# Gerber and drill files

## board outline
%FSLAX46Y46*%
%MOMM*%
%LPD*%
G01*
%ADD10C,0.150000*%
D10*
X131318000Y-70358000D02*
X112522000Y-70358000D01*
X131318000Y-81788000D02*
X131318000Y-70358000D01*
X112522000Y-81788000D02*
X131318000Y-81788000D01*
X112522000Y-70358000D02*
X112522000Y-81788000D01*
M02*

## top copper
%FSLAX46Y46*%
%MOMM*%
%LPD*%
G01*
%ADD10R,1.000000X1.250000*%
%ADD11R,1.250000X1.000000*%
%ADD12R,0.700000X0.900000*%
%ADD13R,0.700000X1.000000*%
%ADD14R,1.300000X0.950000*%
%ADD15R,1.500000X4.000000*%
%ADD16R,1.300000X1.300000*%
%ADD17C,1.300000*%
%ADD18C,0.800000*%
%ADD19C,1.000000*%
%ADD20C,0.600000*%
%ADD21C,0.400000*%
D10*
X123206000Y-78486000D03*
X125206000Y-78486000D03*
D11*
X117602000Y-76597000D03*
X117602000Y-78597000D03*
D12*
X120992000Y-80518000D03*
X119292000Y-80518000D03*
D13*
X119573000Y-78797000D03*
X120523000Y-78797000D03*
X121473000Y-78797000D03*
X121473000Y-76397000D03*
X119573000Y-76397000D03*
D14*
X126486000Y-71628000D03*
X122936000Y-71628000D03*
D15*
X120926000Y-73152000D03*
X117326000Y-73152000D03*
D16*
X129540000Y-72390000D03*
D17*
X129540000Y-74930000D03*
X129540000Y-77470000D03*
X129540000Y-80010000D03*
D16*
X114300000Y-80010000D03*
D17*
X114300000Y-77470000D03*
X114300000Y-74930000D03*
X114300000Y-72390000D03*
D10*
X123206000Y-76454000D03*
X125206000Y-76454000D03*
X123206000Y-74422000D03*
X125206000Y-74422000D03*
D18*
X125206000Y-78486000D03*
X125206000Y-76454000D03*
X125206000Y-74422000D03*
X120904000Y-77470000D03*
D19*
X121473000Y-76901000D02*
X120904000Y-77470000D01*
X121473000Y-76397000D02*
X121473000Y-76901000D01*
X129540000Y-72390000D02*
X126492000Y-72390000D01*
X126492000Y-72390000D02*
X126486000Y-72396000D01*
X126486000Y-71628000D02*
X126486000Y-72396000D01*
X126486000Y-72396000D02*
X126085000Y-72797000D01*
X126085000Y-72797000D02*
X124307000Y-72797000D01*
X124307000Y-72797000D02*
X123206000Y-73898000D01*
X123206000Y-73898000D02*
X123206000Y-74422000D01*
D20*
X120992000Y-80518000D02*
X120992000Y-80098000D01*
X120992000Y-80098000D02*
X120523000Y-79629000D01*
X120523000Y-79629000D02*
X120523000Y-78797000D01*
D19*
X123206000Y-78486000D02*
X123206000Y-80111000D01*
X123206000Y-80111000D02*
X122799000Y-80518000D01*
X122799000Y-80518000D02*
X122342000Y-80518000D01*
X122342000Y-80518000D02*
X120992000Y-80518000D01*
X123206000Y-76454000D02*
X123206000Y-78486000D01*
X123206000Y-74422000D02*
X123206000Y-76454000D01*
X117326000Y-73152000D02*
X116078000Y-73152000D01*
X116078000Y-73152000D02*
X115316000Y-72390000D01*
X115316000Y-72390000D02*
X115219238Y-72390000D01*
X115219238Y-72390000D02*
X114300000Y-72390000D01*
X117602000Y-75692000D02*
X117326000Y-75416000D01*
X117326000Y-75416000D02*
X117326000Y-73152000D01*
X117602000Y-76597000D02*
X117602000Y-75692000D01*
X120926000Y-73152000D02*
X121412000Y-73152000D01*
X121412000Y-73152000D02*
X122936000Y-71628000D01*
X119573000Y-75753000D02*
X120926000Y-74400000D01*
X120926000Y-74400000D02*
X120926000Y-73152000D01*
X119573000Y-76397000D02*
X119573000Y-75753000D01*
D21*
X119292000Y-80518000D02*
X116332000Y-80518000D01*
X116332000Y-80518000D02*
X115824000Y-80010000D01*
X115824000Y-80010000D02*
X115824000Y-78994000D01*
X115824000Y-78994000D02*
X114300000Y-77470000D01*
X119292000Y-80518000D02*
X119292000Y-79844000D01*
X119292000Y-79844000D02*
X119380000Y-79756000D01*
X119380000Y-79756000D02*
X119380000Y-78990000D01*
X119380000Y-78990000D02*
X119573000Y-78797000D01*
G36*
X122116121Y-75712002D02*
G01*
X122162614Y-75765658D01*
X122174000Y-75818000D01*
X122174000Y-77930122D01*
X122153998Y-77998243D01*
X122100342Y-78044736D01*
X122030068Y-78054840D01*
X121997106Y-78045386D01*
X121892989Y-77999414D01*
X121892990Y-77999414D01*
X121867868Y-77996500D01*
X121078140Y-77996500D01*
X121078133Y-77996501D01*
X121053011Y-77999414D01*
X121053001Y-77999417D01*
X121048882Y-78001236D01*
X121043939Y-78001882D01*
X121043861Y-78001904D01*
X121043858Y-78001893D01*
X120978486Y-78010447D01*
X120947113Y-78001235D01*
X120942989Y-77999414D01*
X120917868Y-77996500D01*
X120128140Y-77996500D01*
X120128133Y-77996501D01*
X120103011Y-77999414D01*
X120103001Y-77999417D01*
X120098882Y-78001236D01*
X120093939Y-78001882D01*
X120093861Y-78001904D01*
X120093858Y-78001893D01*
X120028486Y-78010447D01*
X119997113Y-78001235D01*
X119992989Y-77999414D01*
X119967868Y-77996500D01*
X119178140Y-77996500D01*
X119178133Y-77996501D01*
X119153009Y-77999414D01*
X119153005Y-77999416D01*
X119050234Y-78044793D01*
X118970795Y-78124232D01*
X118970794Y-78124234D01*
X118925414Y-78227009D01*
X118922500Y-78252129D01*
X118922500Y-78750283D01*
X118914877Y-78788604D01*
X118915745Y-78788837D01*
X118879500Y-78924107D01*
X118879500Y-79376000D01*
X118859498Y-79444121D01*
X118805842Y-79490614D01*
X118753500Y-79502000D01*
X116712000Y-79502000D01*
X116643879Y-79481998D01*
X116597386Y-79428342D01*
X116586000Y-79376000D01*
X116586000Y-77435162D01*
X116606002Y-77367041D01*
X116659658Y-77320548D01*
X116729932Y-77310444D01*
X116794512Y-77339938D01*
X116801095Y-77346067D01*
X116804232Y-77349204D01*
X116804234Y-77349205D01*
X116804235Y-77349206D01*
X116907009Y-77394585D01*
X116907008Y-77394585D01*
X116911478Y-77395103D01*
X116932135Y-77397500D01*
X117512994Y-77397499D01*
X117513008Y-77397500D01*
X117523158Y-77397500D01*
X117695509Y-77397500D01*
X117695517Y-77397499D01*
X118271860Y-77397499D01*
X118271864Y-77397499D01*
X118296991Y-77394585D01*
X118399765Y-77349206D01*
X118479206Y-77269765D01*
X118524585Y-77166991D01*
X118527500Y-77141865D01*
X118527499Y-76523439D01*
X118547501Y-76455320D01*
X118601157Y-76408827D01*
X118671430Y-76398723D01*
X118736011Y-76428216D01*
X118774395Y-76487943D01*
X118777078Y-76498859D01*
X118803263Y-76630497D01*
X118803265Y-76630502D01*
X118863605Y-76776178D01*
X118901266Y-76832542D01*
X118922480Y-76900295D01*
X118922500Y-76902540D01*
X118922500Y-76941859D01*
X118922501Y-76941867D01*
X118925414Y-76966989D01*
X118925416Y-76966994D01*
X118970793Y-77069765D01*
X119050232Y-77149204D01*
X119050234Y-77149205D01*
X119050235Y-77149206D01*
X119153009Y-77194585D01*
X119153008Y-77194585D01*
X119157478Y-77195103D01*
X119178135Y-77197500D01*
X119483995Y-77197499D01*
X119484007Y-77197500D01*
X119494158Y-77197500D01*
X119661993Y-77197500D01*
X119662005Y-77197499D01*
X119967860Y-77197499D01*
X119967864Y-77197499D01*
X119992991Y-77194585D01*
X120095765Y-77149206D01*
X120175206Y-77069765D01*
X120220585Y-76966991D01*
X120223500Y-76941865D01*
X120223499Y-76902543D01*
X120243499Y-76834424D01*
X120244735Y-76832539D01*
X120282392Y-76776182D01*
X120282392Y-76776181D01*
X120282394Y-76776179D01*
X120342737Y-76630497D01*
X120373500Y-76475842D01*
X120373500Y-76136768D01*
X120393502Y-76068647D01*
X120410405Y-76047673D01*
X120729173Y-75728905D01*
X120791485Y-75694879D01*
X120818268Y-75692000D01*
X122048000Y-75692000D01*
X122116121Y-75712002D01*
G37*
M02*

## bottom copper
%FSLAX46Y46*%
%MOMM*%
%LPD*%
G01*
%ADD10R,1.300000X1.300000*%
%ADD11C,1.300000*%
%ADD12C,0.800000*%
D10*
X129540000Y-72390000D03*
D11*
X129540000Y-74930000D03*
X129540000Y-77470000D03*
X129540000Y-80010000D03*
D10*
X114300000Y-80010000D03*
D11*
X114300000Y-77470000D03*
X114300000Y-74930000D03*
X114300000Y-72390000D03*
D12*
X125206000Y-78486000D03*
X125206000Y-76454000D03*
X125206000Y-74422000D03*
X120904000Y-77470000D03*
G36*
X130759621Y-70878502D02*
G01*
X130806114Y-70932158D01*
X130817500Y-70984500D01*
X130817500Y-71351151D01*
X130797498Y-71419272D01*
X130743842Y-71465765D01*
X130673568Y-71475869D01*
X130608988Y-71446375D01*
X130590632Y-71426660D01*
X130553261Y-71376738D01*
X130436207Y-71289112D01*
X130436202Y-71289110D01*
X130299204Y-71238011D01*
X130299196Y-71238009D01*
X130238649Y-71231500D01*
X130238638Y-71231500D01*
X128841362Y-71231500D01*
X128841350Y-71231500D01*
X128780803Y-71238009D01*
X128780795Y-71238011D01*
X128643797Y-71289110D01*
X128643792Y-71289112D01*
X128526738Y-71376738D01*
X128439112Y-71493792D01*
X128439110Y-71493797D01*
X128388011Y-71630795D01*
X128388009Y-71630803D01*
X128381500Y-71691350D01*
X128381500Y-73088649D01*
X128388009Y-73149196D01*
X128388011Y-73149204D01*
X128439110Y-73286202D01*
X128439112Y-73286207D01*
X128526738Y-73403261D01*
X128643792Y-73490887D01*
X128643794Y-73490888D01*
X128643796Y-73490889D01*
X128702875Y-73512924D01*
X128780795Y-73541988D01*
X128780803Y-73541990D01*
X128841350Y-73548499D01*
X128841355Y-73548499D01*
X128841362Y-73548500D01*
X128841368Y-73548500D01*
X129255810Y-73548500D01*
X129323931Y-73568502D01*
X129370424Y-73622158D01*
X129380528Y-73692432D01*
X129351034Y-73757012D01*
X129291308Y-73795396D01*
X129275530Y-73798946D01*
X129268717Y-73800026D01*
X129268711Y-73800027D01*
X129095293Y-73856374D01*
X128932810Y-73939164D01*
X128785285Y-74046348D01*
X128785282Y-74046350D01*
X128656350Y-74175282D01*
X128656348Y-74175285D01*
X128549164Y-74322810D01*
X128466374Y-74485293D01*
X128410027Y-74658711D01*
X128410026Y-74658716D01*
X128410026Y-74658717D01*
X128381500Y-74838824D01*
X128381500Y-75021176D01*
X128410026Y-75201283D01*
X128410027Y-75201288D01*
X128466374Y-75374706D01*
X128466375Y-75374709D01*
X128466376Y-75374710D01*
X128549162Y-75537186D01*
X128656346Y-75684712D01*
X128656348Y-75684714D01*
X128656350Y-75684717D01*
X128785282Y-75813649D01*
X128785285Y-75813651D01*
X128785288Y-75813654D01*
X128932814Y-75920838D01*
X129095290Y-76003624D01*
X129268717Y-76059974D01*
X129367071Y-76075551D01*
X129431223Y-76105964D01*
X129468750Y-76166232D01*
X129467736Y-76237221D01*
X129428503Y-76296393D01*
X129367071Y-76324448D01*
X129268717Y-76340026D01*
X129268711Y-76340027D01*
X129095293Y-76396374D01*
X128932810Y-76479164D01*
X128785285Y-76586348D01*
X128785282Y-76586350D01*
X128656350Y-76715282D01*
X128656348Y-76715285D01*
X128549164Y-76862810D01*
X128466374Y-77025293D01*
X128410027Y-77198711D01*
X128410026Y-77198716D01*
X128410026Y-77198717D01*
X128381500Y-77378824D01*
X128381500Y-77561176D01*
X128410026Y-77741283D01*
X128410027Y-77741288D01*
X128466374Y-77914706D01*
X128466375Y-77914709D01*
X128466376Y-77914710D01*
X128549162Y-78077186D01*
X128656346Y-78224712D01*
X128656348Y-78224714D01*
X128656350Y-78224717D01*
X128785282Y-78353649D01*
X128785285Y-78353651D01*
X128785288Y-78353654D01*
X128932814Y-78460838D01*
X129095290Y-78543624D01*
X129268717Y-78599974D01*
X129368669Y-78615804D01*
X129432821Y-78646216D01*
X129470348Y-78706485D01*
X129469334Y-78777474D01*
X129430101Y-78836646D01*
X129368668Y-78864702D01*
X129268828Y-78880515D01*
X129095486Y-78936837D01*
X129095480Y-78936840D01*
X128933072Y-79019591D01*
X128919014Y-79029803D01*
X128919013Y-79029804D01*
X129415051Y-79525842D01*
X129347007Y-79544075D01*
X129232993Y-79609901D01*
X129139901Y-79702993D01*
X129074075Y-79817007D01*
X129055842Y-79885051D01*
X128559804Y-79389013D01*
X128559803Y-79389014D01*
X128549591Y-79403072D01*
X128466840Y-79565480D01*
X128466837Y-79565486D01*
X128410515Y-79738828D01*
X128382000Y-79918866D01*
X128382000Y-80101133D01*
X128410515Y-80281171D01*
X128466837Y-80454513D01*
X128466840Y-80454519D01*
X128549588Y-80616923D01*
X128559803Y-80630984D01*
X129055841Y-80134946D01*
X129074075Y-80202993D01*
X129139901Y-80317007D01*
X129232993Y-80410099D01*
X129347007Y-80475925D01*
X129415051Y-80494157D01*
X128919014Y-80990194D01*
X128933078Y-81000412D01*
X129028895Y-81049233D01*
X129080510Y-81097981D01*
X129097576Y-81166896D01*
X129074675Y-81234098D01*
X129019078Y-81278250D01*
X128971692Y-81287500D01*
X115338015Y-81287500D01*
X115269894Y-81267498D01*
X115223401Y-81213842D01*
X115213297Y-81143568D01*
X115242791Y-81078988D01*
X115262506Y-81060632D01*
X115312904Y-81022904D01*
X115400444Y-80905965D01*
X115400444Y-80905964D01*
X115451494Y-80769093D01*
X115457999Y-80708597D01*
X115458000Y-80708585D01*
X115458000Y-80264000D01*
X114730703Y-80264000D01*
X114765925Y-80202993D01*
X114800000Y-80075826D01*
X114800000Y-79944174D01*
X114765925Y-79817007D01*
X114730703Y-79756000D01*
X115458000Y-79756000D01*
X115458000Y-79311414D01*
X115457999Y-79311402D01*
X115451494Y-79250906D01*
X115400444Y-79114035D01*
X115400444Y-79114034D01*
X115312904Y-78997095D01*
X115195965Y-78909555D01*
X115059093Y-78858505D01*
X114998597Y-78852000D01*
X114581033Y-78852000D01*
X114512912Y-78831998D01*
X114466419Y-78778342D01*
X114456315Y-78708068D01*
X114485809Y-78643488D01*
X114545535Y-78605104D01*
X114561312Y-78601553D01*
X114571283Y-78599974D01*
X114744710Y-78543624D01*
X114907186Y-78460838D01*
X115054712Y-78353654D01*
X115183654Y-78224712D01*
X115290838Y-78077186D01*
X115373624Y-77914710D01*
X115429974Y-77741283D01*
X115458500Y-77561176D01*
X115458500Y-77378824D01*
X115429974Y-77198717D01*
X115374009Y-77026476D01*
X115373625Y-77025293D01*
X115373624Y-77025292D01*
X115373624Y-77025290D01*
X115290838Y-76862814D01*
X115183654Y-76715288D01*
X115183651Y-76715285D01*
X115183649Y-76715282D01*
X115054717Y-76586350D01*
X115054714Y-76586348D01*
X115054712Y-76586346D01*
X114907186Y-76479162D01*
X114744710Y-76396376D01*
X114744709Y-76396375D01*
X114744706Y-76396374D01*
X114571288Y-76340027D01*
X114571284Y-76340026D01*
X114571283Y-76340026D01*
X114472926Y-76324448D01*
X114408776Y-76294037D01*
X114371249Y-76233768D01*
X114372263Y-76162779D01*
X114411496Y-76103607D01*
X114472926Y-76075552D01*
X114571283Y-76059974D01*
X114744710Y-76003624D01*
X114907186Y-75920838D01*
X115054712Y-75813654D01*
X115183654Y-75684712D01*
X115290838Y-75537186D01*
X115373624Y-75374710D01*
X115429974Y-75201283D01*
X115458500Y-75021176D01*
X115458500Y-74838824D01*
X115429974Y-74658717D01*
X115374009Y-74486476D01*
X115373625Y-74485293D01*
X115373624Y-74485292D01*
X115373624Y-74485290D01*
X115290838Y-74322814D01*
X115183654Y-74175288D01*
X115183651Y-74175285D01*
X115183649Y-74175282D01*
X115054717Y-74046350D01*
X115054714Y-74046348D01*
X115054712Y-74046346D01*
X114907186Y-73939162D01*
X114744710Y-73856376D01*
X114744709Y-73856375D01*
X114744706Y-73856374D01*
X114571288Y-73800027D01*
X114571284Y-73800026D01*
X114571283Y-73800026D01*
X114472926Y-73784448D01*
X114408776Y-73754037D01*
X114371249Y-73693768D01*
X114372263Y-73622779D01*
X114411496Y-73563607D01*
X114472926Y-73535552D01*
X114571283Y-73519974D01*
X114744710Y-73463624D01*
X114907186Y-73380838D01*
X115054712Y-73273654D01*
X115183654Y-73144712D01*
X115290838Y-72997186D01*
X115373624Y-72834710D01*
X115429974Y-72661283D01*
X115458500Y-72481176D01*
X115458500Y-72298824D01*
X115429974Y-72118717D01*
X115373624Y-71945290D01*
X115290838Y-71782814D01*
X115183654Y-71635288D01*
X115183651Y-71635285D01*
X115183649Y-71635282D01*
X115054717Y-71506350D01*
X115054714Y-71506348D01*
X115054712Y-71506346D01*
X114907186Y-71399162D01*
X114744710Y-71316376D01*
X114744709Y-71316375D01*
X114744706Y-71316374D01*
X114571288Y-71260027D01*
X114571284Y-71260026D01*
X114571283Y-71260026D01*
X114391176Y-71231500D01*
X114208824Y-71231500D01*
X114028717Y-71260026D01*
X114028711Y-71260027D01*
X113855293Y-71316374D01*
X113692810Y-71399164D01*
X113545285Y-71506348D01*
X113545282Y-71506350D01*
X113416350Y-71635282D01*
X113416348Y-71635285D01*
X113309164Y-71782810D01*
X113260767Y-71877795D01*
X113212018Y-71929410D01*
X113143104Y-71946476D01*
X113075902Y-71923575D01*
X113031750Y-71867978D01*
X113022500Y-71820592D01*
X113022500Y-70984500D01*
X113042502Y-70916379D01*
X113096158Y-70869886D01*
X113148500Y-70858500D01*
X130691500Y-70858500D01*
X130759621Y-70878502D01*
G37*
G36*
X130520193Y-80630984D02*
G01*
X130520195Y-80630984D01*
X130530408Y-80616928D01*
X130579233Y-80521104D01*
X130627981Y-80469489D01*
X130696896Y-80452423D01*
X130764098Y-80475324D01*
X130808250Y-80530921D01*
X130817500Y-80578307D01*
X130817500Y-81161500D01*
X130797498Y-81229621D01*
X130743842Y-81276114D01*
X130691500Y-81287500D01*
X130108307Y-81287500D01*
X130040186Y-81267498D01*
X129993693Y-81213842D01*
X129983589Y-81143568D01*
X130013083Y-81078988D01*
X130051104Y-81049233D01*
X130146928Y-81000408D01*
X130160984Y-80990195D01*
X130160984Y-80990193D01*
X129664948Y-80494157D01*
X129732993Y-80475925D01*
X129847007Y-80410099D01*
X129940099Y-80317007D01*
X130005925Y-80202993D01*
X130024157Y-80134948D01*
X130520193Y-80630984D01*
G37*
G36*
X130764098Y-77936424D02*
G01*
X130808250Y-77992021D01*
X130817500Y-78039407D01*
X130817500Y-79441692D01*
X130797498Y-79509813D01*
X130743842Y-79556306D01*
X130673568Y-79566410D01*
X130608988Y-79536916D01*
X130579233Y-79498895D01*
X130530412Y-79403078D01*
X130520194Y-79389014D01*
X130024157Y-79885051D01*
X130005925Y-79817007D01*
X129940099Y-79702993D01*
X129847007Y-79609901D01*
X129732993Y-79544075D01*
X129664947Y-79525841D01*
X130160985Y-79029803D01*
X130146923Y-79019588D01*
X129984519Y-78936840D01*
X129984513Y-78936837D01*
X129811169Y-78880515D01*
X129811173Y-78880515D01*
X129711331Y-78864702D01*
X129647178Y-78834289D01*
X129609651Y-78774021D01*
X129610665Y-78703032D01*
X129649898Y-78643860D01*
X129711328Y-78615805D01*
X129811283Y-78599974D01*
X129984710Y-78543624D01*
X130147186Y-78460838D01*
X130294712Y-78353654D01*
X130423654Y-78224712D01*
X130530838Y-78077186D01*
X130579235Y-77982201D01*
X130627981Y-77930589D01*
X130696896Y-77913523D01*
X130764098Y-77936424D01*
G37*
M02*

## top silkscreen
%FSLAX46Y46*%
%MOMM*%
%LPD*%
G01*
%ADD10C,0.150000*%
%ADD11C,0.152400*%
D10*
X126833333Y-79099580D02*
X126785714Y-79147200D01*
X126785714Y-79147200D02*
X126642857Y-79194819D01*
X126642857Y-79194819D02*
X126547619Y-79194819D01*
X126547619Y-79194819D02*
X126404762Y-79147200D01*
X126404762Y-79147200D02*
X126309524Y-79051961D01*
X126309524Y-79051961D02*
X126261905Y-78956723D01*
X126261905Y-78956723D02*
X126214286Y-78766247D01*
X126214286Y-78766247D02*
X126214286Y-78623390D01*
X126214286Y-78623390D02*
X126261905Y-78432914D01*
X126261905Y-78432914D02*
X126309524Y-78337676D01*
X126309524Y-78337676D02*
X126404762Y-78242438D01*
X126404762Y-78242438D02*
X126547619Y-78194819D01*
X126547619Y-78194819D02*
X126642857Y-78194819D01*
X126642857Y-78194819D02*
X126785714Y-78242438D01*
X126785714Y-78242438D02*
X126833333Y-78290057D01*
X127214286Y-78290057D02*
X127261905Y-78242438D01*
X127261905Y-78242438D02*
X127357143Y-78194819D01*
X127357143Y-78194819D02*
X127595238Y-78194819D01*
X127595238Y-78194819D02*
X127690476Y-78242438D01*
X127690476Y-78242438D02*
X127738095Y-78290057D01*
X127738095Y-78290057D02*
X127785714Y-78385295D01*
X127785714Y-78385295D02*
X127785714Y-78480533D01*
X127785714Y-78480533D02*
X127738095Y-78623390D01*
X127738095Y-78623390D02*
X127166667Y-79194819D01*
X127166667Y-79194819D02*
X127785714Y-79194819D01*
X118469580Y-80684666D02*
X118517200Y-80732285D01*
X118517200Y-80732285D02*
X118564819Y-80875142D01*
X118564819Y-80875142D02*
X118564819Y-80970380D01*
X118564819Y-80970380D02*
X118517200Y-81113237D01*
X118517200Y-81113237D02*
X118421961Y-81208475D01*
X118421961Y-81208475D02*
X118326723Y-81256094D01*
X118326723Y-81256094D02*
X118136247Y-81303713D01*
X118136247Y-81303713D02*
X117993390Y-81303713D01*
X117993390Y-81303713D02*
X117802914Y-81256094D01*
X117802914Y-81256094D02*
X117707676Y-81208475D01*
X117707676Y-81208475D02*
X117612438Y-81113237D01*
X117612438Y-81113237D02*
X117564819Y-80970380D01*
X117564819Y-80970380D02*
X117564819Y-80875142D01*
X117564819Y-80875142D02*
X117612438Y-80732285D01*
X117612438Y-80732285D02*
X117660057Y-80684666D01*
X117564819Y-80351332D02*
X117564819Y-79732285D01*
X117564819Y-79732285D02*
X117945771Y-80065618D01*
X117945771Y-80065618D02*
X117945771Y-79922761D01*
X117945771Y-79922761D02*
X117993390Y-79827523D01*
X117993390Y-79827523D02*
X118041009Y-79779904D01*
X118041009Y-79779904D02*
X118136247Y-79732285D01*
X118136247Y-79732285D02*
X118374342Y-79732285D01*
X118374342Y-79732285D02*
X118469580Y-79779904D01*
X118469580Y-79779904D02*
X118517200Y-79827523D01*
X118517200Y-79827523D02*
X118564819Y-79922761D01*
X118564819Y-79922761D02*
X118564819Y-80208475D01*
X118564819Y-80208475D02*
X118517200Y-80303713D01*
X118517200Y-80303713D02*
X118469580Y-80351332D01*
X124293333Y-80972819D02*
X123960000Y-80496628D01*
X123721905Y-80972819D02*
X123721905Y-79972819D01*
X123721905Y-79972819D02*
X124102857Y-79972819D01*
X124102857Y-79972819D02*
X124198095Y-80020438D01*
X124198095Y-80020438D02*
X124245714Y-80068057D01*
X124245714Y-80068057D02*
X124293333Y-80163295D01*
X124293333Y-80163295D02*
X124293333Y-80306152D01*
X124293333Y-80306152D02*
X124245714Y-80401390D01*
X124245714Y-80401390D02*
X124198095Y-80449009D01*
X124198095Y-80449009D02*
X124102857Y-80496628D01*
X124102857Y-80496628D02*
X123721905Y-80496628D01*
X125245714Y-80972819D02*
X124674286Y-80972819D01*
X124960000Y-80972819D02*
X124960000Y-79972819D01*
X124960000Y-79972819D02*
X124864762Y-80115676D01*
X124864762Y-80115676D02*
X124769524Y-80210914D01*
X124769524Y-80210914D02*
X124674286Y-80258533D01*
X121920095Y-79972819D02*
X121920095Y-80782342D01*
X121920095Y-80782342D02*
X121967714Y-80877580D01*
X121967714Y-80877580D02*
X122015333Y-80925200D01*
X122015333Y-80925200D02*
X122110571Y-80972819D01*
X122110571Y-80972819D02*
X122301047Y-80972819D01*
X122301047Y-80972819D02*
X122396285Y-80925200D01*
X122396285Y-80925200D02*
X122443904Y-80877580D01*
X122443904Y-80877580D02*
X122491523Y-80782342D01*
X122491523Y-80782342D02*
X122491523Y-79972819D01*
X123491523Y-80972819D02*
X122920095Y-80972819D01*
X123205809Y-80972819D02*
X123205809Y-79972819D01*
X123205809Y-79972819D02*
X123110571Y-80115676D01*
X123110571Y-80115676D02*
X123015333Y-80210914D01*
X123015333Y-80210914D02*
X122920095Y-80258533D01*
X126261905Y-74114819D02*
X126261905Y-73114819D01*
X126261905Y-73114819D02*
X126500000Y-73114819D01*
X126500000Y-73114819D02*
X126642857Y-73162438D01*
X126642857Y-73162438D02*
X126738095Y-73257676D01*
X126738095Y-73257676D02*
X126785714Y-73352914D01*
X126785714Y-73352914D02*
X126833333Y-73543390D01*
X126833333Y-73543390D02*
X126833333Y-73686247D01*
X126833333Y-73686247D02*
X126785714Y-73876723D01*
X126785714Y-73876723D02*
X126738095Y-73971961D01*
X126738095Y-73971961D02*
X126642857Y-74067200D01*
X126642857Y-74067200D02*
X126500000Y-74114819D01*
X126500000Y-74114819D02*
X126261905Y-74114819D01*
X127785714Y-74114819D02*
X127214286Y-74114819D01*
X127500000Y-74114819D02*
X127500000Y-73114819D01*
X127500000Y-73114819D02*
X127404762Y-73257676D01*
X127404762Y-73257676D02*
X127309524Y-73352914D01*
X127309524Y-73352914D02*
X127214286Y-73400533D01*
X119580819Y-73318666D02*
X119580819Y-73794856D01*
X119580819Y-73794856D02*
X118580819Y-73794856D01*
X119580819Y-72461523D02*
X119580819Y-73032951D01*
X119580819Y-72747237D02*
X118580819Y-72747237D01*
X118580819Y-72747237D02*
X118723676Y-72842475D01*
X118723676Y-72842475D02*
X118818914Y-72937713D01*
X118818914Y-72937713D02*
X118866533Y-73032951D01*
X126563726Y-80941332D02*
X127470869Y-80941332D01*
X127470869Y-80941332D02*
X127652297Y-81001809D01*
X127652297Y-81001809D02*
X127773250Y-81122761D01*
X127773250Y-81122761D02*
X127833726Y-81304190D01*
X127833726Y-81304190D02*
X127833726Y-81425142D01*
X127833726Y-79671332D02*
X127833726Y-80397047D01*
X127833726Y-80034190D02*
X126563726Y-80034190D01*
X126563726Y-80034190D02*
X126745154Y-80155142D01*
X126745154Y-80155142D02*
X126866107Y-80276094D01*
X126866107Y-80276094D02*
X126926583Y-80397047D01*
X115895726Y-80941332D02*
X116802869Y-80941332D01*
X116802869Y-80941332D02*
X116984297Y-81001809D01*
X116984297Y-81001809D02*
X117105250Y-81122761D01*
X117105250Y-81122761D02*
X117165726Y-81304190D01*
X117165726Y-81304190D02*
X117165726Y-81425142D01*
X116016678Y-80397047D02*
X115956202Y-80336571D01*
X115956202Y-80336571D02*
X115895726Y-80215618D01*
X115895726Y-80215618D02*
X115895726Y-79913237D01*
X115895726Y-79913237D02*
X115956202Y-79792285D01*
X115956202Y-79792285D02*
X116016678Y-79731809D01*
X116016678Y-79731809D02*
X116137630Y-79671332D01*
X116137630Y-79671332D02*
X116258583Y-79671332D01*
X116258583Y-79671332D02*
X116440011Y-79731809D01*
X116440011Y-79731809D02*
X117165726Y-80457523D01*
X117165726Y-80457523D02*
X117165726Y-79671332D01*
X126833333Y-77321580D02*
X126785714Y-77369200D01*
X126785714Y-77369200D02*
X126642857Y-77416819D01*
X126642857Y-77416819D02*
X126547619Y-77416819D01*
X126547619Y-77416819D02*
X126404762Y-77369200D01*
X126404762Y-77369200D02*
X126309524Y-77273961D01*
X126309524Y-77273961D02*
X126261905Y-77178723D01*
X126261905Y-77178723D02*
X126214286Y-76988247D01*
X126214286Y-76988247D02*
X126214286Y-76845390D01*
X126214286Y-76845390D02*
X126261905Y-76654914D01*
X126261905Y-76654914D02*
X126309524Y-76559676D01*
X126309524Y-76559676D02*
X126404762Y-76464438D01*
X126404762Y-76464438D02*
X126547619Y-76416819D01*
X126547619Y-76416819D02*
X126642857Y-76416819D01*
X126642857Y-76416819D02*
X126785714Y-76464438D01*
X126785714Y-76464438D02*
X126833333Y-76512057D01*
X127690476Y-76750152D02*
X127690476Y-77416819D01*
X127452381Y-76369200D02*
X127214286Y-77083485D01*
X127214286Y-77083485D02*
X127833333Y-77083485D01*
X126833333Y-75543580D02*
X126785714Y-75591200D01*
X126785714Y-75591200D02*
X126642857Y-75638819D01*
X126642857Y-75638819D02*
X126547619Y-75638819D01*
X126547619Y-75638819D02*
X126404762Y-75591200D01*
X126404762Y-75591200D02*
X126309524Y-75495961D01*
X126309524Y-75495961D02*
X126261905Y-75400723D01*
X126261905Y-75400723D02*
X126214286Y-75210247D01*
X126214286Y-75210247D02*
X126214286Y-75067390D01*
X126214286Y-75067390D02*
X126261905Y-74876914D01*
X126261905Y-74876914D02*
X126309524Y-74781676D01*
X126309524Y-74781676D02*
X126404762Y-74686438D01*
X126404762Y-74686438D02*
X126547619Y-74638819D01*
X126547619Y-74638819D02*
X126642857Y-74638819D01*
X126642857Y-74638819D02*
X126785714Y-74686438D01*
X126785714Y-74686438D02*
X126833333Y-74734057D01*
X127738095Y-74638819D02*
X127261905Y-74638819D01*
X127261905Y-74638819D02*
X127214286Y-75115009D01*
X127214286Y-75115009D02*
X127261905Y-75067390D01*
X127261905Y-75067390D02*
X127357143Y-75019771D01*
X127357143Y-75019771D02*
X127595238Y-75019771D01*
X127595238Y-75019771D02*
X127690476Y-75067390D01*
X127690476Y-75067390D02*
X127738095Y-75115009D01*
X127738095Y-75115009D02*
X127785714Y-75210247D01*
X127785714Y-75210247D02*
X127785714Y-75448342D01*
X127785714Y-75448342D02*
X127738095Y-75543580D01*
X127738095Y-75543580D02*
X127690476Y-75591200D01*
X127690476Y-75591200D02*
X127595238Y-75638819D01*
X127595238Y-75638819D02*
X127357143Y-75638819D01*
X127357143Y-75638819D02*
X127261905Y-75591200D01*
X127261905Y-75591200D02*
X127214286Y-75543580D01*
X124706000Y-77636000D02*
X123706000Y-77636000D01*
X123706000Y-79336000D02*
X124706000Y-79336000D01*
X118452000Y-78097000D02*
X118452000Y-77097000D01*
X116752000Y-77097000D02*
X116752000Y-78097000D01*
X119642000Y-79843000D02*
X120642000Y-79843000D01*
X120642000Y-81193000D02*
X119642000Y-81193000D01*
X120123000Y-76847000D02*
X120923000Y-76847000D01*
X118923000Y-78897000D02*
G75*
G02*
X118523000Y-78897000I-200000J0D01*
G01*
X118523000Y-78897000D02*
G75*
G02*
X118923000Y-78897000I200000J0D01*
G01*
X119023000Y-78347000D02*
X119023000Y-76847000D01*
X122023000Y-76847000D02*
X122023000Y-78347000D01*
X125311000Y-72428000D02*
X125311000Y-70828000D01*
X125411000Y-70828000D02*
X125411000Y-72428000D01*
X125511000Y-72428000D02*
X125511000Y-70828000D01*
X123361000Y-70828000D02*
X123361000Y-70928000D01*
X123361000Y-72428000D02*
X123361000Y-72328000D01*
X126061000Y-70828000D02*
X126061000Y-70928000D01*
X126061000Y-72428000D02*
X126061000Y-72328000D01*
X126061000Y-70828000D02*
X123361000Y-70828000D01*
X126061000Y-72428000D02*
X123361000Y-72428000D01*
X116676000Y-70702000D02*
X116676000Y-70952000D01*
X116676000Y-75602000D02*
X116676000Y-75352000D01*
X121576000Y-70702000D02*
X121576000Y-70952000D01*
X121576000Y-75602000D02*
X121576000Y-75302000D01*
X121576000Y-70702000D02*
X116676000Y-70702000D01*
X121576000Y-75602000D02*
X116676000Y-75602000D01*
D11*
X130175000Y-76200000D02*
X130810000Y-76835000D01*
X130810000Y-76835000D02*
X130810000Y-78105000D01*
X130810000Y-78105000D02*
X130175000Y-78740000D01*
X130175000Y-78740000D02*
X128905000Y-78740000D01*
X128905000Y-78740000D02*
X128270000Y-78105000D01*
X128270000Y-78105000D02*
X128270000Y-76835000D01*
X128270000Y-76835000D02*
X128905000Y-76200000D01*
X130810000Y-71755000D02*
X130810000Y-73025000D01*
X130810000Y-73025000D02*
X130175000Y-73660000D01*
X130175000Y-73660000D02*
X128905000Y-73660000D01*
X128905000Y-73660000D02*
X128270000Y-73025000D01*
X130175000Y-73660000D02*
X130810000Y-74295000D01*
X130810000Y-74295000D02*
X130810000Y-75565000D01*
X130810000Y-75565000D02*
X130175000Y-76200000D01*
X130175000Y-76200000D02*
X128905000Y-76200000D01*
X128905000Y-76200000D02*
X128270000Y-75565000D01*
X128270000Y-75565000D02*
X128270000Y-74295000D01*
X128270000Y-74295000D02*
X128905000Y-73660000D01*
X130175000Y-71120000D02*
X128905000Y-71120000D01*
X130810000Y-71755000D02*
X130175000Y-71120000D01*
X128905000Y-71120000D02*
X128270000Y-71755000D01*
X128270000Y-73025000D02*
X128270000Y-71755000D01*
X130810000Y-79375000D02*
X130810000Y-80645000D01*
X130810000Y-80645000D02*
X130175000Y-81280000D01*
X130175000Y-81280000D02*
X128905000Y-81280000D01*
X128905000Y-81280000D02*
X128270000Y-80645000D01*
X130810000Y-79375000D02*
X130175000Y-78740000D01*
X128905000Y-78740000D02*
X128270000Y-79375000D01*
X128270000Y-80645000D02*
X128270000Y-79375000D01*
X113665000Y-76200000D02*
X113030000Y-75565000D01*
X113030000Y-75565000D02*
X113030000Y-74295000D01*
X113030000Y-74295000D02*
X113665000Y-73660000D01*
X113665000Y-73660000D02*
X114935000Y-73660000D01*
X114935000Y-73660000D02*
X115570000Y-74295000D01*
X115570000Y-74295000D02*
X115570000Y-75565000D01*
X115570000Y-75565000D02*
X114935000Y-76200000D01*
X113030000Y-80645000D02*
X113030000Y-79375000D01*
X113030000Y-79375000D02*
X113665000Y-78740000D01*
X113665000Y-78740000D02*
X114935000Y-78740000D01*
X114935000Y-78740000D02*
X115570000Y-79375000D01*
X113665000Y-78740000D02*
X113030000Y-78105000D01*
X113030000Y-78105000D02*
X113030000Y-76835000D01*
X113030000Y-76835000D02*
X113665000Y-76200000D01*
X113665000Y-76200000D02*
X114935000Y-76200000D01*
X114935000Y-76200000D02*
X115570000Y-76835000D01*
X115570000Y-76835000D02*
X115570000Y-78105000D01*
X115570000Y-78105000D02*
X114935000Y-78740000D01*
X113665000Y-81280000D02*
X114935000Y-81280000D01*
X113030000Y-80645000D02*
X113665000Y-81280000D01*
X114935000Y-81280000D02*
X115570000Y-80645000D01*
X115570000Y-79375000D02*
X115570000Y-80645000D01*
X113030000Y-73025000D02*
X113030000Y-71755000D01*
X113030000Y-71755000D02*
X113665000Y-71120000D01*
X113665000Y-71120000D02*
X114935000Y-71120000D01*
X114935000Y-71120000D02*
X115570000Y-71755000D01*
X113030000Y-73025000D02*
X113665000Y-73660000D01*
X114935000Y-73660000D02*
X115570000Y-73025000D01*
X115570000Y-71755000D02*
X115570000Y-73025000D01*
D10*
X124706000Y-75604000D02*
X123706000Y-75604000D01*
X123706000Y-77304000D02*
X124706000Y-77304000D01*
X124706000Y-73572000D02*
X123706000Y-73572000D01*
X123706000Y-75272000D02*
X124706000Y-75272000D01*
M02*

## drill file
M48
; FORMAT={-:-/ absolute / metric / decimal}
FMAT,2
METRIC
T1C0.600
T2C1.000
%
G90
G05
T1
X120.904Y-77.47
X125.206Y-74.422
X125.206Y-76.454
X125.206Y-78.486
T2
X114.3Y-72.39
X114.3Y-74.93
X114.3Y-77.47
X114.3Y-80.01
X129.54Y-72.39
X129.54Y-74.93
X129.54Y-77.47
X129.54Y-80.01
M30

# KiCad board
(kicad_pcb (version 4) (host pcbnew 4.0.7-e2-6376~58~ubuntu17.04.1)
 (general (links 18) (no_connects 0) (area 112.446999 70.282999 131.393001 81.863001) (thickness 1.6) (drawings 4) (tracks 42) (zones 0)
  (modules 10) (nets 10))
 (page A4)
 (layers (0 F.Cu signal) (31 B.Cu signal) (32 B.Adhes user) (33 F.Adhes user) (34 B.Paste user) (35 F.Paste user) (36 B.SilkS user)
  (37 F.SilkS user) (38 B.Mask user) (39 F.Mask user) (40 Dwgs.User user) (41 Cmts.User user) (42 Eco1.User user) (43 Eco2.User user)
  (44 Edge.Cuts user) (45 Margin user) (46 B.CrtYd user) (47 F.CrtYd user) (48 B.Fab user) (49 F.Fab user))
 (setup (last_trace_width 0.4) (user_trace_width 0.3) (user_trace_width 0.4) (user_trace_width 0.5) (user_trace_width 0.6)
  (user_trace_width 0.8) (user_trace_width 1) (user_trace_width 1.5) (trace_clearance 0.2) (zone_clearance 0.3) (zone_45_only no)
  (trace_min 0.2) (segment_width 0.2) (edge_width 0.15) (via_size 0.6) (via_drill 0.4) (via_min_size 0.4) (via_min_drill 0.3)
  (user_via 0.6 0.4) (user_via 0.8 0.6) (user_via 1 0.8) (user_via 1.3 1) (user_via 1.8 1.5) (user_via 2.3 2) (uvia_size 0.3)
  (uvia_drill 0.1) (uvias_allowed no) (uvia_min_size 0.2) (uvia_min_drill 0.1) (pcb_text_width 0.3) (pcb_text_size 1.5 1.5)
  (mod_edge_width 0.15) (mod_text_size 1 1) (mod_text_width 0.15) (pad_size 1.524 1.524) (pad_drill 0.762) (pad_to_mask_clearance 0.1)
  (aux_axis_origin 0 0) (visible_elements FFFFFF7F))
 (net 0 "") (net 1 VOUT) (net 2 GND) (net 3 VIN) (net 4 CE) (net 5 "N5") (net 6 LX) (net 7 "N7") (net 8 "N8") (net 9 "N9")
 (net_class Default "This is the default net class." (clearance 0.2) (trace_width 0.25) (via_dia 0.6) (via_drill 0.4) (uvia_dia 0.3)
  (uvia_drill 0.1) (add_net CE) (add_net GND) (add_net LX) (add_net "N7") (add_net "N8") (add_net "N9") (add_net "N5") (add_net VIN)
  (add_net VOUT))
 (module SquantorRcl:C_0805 (layer F.Cu) (at 124.206 78.486)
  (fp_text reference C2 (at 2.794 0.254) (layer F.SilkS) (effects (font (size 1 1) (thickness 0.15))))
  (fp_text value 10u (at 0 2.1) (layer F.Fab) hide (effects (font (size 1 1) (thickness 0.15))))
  (fp_line (start 0.5 -0.85) (end -0.5 -0.85) (layer F.SilkS) (width 0.15))
  (fp_line (start -0.5 0.85) (end 0.5 0.85) (layer F.SilkS) (width 0.15))
  (pad 1 smd rect (at -1 0) (size 1 1.25) (layers F.Cu F.Paste F.Mask) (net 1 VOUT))
  (pad 2 smd rect (at 1 0) (size 1 1.25) (layers F.Cu F.Paste F.Mask) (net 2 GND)))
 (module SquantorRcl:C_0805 (layer F.Cu) (at 117.602 77.597 270)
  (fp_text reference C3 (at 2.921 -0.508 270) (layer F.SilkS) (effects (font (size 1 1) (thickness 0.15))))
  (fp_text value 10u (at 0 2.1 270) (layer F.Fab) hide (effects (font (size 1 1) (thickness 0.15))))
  (fp_line (start 0.5 -0.85) (end -0.5 -0.85) (layer F.SilkS) (width 0.15))
  (fp_line (start -0.5 0.85) (end 0.5 0.85) (layer F.SilkS) (width 0.15))
  (pad 1 smd rect (at -1 0 270) (size 1 1.25) (layers F.Cu F.Paste F.Mask) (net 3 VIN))
  (pad 2 smd rect (at 1 0 270) (size 1 1.25) (layers F.Cu F.Paste F.Mask) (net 2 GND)))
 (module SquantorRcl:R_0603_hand (layer F.Cu) (at 120.142 80.518 180)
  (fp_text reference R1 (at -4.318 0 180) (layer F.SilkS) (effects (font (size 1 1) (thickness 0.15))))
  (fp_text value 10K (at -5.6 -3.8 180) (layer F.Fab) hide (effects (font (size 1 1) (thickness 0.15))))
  (fp_line (start 0.5 0.675) (end -0.5 0.675) (layer F.SilkS) (width 0.15))
  (fp_line (start -0.5 -0.675) (end 0.5 -0.675) (layer F.SilkS) (width 0.15))
  (pad 1 smd rect (at -0.85 0 180) (size 0.7 0.9) (layers F.Cu F.Paste F.Mask) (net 1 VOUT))
  (pad 2 smd rect (at 0.85 0 180) (size 0.7 0.9) (layers F.Cu F.Paste F.Mask) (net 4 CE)))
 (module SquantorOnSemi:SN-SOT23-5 (layer F.Cu) (at 120.523 77.597)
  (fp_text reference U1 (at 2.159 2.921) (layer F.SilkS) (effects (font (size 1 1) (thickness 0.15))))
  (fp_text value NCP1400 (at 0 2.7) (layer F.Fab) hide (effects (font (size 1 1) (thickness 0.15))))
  (fp_line (start -0.4 -0.75) (end 0.4 -0.75) (layer F.SilkS) (width 0.15))
  (fp_circle (center -1.8 1.3) (end -1.6 1.3) (layer F.SilkS) (width 0.15))
  (fp_line (start -1.5 0.75) (end -1.5 -0.75) (layer F.SilkS) (width 0.15))
  (fp_line (start 1.5 -0.75) (end 1.5 0.75) (layer F.SilkS) (width 0.15))
  (pad 1 smd rect (at -0.95 1.2) (size 0.7 1) (layers F.Cu F.Paste F.Mask) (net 4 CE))
  (pad 2 smd rect (at 0 1.2) (size 0.7 1) (layers F.Cu F.Paste F.Mask) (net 1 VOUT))
  (pad 3 smd rect (at 0.95 1.2) (size 0.7 1) (layers F.Cu F.Paste F.Mask) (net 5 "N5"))
  (pad 4 smd rect (at 0.95 -1.2) (size 0.7 1) (layers F.Cu F.Paste F.Mask) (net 2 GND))
  (pad 5 smd rect (at -0.95 -1.2) (size 0.7 1) (layers F.Cu F.Paste F.Mask) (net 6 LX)))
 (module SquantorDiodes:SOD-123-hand (layer F.Cu) (at 124.711 71.628 180)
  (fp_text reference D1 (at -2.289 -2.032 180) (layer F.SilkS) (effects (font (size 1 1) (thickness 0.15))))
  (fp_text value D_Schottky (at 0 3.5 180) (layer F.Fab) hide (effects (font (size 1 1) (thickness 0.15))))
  (fp_line (start -0.6 -0.8) (end -0.6 0.8) (layer F.SilkS) (width 0.15))
  (fp_line (start -0.7 0.8) (end -0.7 -0.8) (layer F.SilkS) (width 0.15))
  (fp_line (start -0.8 -0.8) (end -0.8 0.8) (layer F.SilkS) (width 0.15))
  (fp_line (start 1.35 0.8) (end 1.35 0.7) (layer F.SilkS) (width 0.15))
  (fp_line (start 1.35 -0.8) (end 1.35 -0.7) (layer F.SilkS) (width 0.15))
  (fp_line (start -1.35 0.8) (end -1.35 0.7) (layer F.SilkS) (width 0.15))
  (fp_line (start -1.35 -0.8) (end -1.35 -0.7) (layer F.SilkS) (width 0.15))
  (fp_line (start -1.35 0.8) (end 1.35 0.8) (layer F.SilkS) (width 0.15))
  (fp_line (start -1.35 -0.8) (end 1.35 -0.8) (layer F.SilkS) (width 0.15))
  (pad 1 smd rect (at -1.775 0 180) (size 1.3 0.95) (layers F.Cu F.Paste F.Mask) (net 1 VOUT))
  (pad 2 smd rect (at 1.775 0 180) (size 1.3 0.95) (layers F.Cu F.Paste F.Mask) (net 6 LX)))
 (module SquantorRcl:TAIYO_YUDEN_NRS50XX (layer F.Cu) (at 119.126 73.152 180)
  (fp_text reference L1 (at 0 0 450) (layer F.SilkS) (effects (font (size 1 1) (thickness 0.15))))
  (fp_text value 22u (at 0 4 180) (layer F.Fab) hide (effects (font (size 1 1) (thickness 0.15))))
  (fp_line (start 2.45 2.45) (end 2.45 2.2) (layer F.SilkS) (width 0.15))
  (fp_line (start 2.45 -2.45) (end 2.45 -2.2) (layer F.SilkS) (width 0.15))
  (fp_line (start -2.45 2.45) (end -2.45 2.2) (layer F.SilkS) (width 0.15))
  (fp_line (start -2.45 -2.45) (end -2.45 -2.15) (layer F.SilkS) (width 0.15))
  (fp_line (start -2.45 2.45) (end 2.45 2.45) (layer F.SilkS) (width 0.15))
  (fp_line (start -2.45 -2.45) (end 2.45 -2.45) (layer F.SilkS) (width 0.15))
  (pad 1 smd rect (at -1.8 0 180) (size 1.5 4) (layers F.Cu F.Paste F.Mask) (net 6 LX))
  (pad 2 smd rect (at 1.8 0 180) (size 1.5 4) (layers F.Cu F.Paste F.Mask) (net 3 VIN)))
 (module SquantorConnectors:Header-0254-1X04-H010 (layer F.Cu) (at 129.54 76.2 270)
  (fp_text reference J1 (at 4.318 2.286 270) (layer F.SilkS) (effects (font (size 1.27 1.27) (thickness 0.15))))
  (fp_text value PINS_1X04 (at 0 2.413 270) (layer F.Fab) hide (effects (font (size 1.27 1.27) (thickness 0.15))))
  (fp_line (start 0 -0.635) (end 0.635 -1.27) (layer F.SilkS) (width 0.1524))
  (fp_line (start 0.635 -1.27) (end 1.905 -1.27) (layer F.SilkS) (width 0.1524))
  (fp_line (start 1.905 -1.27) (end 2.54 -0.635) (layer F.SilkS) (width 0.1524))
  (fp_line (start 2.54 -0.635) (end 2.54 0.635) (layer F.SilkS) (width 0.1524))
  (fp_line (start 2.54 0.635) (end 1.905 1.27) (layer F.SilkS) (width 0.1524))
  (fp_line (start 1.905 1.27) (end 0.635 1.27) (layer F.SilkS) (width 0.1524))
  (fp_line (start 0.635 1.27) (end 0 0.635) (layer F.SilkS) (width 0.1524))
  (fp_line (start -4.445 -1.27) (end -3.175 -1.27) (layer F.SilkS) (width 0.1524))
  (fp_line (start -3.175 -1.27) (end -2.54 -0.635) (layer F.SilkS) (width 0.1524))
  (fp_line (start -2.54 -0.635) (end -2.54 0.635) (layer F.SilkS) (width 0.1524))
  (fp_line (start -2.54 0.635) (end -3.175 1.27) (layer F.SilkS) (width 0.1524))
  (fp_line (start -2.54 -0.635) (end -1.905 -1.27) (layer F.SilkS) (width 0.1524))
  (fp_line (start -1.905 -1.27) (end -0.635 -1.27) (layer F.SilkS) (width 0.1524))
  (fp_line (start -0.635 -1.27) (end 0 -0.635) (layer F.SilkS) (width 0.1524))
  (fp_line (start 0 -0.635) (end 0 0.635) (layer F.SilkS) (width 0.1524))
  (fp_line (start 0 0.635) (end -0.635 1.27) (layer F.SilkS) (width 0.1524))
  (fp_line (start -0.635 1.27) (end -1.905 1.27) (layer F.SilkS) (width 0.1524))
  (fp_line (start -1.905 1.27) (end -2.54 0.635) (layer F.SilkS) (width 0.1524))
  (fp_line (start -5.08 -0.635) (end -5.08 0.635) (layer F.SilkS) (width 0.1524))
  (fp_line (start -4.445 -1.27) (end -5.08 -0.635) (layer F.SilkS) (width 0.1524))
  (fp_line (start -5.08 0.635) (end -4.445 1.27) (layer F.SilkS) (width 0.1524))
  (fp_line (start -3.175 1.27) (end -4.445 1.27) (layer F.SilkS) (width 0.1524))
  (fp_line (start 3.175 -1.27) (end 4.445 -1.27) (layer F.SilkS) (width 0.1524))
  (fp_line (start 4.445 -1.27) (end 5.08 -0.635) (layer F.SilkS) (width 0.1524))
  (fp_line (start 5.08 -0.635) (end 5.08 0.635) (layer F.SilkS) (width 0.1524))
  (fp_line (start 5.08 0.635) (end 4.445 1.27) (layer F.SilkS) (width 0.1524))
  (fp_line (start 3.175 -1.27) (end 2.54 -0.635) (layer F.SilkS) (width 0.1524))
  (fp_line (start 2.54 0.635) (end 3.175 1.27) (layer F.SilkS) (width 0.1524))
  (fp_line (start 4.445 1.27) (end 3.175 1.27) (layer F.SilkS) (width 0.1524))
  (pad 1 thru_hole rect (at -3.81 0 90) (size 1.3 1.3) (drill 1) (layers *.Cu *.Mask) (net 1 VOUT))
  (pad 2 thru_hole circle (at -1.27 0 90) (size 1.3 1.3) (drill 1) (layers *.Cu *.Mask) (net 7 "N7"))
  (pad 3 thru_hole circle (at 1.27 0 90) (size 1.3 1.3) (drill 1) (layers *.Cu *.Mask) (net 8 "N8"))
  (pad 4 thru_hole circle (at 3.81 0 90) (size 1.3 1.3) (drill 1) (layers *.Cu *.Mask) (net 2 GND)))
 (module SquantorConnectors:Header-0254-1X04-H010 (layer F.Cu) (at 114.3 76.2 90)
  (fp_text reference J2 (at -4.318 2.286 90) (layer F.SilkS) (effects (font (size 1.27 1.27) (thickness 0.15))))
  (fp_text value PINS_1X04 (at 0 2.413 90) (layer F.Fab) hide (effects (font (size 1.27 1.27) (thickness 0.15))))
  (fp_line (start 0 -0.635) (end 0.635 -1.27) (layer F.SilkS) (width 0.1524))
  (fp_line (start 0.635 -1.27) (end 1.905 -1.27) (layer F.SilkS) (width 0.1524))
  (fp_line (start 1.905 -1.27) (end 2.54 -0.635) (layer F.SilkS) (width 0.1524))
  (fp_line (start 2.54 -0.635) (end 2.54 0.635) (layer F.SilkS) (width 0.1524))
  (fp_line (start 2.54 0.635) (end 1.905 1.27) (layer F.SilkS) (width 0.1524))
  (fp_line (start 1.905 1.27) (end 0.635 1.27) (layer F.SilkS) (width 0.1524))
  (fp_line (start 0.635 1.27) (end 0 0.635) (layer F.SilkS) (width 0.1524))
  (fp_line (start -4.445 -1.27) (end -3.175 -1.27) (layer F.SilkS) (width 0.1524))
  (fp_line (start -3.175 -1.27) (end -2.54 -0.635) (layer F.SilkS) (width 0.1524))
  (fp_line (start -2.54 -0.635) (end -2.54 0.635) (layer F.SilkS) (width 0.1524))
  (fp_line (start -2.54 0.635) (end -3.175 1.27) (layer F.SilkS) (width 0.1524))
  (fp_line (start -2.54 -0.635) (end -1.905 -1.27) (layer F.SilkS) (width 0.1524))
  (fp_line (start -1.905 -1.27) (end -0.635 -1.27) (layer F.SilkS) (width 0.1524))
  (fp_line (start -0.635 -1.27) (end 0 -0.635) (layer F.SilkS) (width 0.1524))
  (fp_line (start 0 -0.635) (end 0 0.635) (layer F.SilkS) (width 0.1524))
  (fp_line (start 0 0.635) (end -0.635 1.27) (layer F.SilkS) (width 0.1524))
  (fp_line (start -0.635 1.27) (end -1.905 1.27) (layer F.SilkS) (width 0.1524))
  (fp_line (start -1.905 1.27) (end -2.54 0.635) (layer F.SilkS) (width 0.1524))
  (fp_line (start -5.08 -0.635) (end -5.08 0.635) (layer F.SilkS) (width 0.1524))
  (fp_line (start -4.445 -1.27) (end -5.08 -0.635) (layer F.SilkS) (width 0.1524))
  (fp_line (start -5.08 0.635) (end -4.445 1.27) (layer F.SilkS) (width 0.1524))
  (fp_line (start -3.175 1.27) (end -4.445 1.27) (layer F.SilkS) (width 0.1524))
  (fp_line (start 3.175 -1.27) (end 4.445 -1.27) (layer F.SilkS) (width 0.1524))
  (fp_line (start 4.445 -1.27) (end 5.08 -0.635) (layer F.SilkS) (width 0.1524))
  (fp_line (start 5.08 -0.635) (end 5.08 0.635) (layer F.SilkS) (width 0.1524))
  (fp_line (start 5.08 0.635) (end 4.445 1.27) (layer F.SilkS) (width 0.1524))
  (fp_line (start 3.175 -1.27) (end 2.54 -0.635) (layer F.SilkS) (width 0.1524))
  (fp_line (start 2.54 0.635) (end 3.175 1.27) (layer F.SilkS) (width 0.1524))
  (fp_line (start 4.445 1.27) (end 3.175 1.27) (layer F.SilkS) (width 0.1524))
  (pad 1 thru_hole rect (at -3.81 0 270) (size 1.3 1.3) (drill 1) (layers *.Cu *.Mask) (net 2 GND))
  (pad 2 thru_hole circle (at -1.27 0 270) (size 1.3 1.3) (drill 1) (layers *.Cu *.Mask) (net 4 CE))
  (pad 3 thru_hole circle (at 1.27 0 270) (size 1.3 1.3) (drill 1) (layers *.Cu *.Mask) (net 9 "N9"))
  (pad 4 thru_hole circle (at 3.81 0 270) (size 1.3 1.3) (drill 1) (layers *.Cu *.Mask) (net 3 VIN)))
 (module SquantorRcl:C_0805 (layer F.Cu) (at 124.206 76.454)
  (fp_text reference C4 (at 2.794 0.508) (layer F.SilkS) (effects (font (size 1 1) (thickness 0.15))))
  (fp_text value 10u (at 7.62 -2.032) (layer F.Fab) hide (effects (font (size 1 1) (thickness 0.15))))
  (fp_line (start 0.5 -0.85) (end -0.5 -0.85) (layer F.SilkS) (width 0.15))
  (fp_line (start -0.5 0.85) (end 0.5 0.85) (layer F.SilkS) (width 0.15))
  (pad 1 smd rect (at -1 0) (size 1 1.25) (layers F.Cu F.Paste F.Mask) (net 1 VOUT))
  (pad 2 smd rect (at 1 0) (size 1 1.25) (layers F.Cu F.Paste F.Mask) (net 2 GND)))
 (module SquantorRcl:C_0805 (layer F.Cu) (at 124.206 74.422)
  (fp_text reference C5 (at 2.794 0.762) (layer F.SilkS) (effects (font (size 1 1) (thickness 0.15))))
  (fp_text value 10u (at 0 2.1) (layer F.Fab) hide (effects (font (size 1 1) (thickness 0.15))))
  (fp_line (start 0.5 -0.85) (end -0.5 -0.85) (layer F.SilkS) (width 0.15))
  (fp_line (start -0.5 0.85) (end 0.5 0.85) (layer F.SilkS) (width 0.15))
  (pad 1 smd rect (at -1 0) (size 1 1.25) (layers F.Cu F.Paste F.Mask) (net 1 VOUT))
  (pad 2 smd rect (at 1 0) (size 1 1.25) (layers F.Cu F.Paste F.Mask) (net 2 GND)))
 (gr_line (start 131.318 70.358) (end 112.522 70.358) (layer Edge.Cuts) (width 0.15))
 (gr_line (start 131.318 81.788) (end 131.318 70.358) (layer Edge.Cuts) (width 0.15))
 (gr_line (start 112.522 81.788) (end 131.318 81.788) (layer Edge.Cuts) (width 0.15))
 (gr_line (start 112.522 70.358) (end 112.522 81.788) (layer Edge.Cuts) (width 0.15))
 (via (at 125.206 78.486) (size 0.8) (drill 0.6) (layers F.Cu B.Cu) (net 2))
 (via (at 125.206 76.454) (size 0.8) (drill 0.6) (layers F.Cu B.Cu) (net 2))
 (via (at 125.206 74.422) (size 0.8) (drill 0.6) (layers F.Cu B.Cu) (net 2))
 (segment (start 121.473 76.901) (end 120.904 77.47) (width 1) (layer F.Cu) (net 2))
 (via (at 120.904 77.47) (size 0.8) (drill 0.6) (layers F.Cu B.Cu) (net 2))
 (segment (start 121.473 76.397) (end 121.473 76.901) (width 1) (layer F.Cu) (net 2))
 (segment (start 129.54 72.39) (end 126.492 72.39) (width 1) (layer F.Cu) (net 1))
 (segment (start 126.492 72.39) (end 126.486 72.396) (width 1) (layer F.Cu) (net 1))
 (segment (start 126.486 71.628) (end 126.486 72.396) (width 1) (layer F.Cu) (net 1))
 (segment (start 126.486 72.396) (end 126.085 72.797) (width 1) (layer F.Cu) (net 1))
 (segment (start 126.085 72.797) (end 124.307 72.797) (width 1) (layer F.Cu) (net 1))
 (segment (start 124.307 72.797) (end 123.206 73.898) (width 1) (layer F.Cu) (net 1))
 (segment (start 123.206 73.898) (end 123.206 74.422) (width 1) (layer F.Cu) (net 1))
 (segment (start 120.992 80.518) (end 120.992 80.098) (width 0.6) (layer F.Cu) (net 1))
 (segment (start 120.992 80.098) (end 120.523 79.629) (width 0.6) (layer F.Cu) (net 1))
 (segment (start 120.523 79.629) (end 120.523 78.797) (width 0.6) (layer F.Cu) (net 1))
 (segment (start 123.206 78.486) (end 123.206 80.111) (width 1) (layer F.Cu) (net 1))
 (segment (start 123.206 80.111) (end 122.799 80.518) (width 1) (layer F.Cu) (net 1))
 (segment (start 122.799 80.518) (end 122.342 80.518) (width 1) (layer F.Cu) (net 1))
 (segment (start 122.342 80.518) (end 120.992 80.518) (width 1) (layer F.Cu) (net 1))
 (segment (start 123.206 76.454) (end 123.206 78.486) (width 1) (layer F.Cu) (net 1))
 (segment (start 123.206 74.422) (end 123.206 76.454) (width 1) (layer F.Cu) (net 1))
 (segment (start 117.326 73.152) (end 116.078 73.152) (width 1) (layer F.Cu) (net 3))
 (segment (start 116.078 73.152) (end 115.316 72.39) (width 1) (layer F.Cu) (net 3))
 (segment (start 115.316 72.39) (end 115.219238 72.39) (width 1) (layer F.Cu) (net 3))
 (segment (start 115.219238 72.39) (end 114.3 72.39) (width 1) (layer F.Cu) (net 3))
 (segment (start 117.602 75.692) (end 117.326 75.416) (width 1) (layer F.Cu) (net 3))
 (segment (start 117.326 75.416) (end 117.326 73.152) (width 1) (layer F.Cu) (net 3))
 (segment (start 117.602 76.597) (end 117.602 75.692) (width 1) (layer F.Cu) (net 3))
 (segment (start 120.926 73.152) (end 121.412 73.152) (width 1) (layer F.Cu) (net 6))
 (segment (start 121.412 73.152) (end 122.936 71.628) (width 1) (layer F.Cu) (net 6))
 (segment (start 119.573 75.753) (end 120.926 74.4) (width 1) (layer F.Cu) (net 6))
 (segment (start 120.926 74.4) (end 120.926 73.152) (width 1) (layer F.Cu) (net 6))
 (segment (start 119.573 76.397) (end 119.573 75.753) (width 1) (layer F.Cu) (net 6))
 (segment (start 119.292 80.518) (end 116.332 80.518) (width 0.4) (layer F.Cu) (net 4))
 (segment (start 116.332 80.518) (end 115.824 80.01) (width 0.4) (layer F.Cu) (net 4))
 (segment (start 115.824 80.01) (end 115.824 78.994) (width 0.4) (layer F.Cu) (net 4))
 (segment (start 115.824 78.994) (end 114.3 77.47) (width 0.4) (layer F.Cu) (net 4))
 (segment (start 119.292 80.518) (end 119.292 79.844) (width 0.4) (layer F.Cu) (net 4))
 (segment (start 119.292 79.844) (end 119.38 79.756) (width 0.4) (layer F.Cu) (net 4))
 (segment (start 119.38 79.756) (end 119.38 78.99) (width 0.4) (layer F.Cu) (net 4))
 (segment (start 119.38 78.99) (end 119.573 78.797) (width 0.4) (layer F.Cu) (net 4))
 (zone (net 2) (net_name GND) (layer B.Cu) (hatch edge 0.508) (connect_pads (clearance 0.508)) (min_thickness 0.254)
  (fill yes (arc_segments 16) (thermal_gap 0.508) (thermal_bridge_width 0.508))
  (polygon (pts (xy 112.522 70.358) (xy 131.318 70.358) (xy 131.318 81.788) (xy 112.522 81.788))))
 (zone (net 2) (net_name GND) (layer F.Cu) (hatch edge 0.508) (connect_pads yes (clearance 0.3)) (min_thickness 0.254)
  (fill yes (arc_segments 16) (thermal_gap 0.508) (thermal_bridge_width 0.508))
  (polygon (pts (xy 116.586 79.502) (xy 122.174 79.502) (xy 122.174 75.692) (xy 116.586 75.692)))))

